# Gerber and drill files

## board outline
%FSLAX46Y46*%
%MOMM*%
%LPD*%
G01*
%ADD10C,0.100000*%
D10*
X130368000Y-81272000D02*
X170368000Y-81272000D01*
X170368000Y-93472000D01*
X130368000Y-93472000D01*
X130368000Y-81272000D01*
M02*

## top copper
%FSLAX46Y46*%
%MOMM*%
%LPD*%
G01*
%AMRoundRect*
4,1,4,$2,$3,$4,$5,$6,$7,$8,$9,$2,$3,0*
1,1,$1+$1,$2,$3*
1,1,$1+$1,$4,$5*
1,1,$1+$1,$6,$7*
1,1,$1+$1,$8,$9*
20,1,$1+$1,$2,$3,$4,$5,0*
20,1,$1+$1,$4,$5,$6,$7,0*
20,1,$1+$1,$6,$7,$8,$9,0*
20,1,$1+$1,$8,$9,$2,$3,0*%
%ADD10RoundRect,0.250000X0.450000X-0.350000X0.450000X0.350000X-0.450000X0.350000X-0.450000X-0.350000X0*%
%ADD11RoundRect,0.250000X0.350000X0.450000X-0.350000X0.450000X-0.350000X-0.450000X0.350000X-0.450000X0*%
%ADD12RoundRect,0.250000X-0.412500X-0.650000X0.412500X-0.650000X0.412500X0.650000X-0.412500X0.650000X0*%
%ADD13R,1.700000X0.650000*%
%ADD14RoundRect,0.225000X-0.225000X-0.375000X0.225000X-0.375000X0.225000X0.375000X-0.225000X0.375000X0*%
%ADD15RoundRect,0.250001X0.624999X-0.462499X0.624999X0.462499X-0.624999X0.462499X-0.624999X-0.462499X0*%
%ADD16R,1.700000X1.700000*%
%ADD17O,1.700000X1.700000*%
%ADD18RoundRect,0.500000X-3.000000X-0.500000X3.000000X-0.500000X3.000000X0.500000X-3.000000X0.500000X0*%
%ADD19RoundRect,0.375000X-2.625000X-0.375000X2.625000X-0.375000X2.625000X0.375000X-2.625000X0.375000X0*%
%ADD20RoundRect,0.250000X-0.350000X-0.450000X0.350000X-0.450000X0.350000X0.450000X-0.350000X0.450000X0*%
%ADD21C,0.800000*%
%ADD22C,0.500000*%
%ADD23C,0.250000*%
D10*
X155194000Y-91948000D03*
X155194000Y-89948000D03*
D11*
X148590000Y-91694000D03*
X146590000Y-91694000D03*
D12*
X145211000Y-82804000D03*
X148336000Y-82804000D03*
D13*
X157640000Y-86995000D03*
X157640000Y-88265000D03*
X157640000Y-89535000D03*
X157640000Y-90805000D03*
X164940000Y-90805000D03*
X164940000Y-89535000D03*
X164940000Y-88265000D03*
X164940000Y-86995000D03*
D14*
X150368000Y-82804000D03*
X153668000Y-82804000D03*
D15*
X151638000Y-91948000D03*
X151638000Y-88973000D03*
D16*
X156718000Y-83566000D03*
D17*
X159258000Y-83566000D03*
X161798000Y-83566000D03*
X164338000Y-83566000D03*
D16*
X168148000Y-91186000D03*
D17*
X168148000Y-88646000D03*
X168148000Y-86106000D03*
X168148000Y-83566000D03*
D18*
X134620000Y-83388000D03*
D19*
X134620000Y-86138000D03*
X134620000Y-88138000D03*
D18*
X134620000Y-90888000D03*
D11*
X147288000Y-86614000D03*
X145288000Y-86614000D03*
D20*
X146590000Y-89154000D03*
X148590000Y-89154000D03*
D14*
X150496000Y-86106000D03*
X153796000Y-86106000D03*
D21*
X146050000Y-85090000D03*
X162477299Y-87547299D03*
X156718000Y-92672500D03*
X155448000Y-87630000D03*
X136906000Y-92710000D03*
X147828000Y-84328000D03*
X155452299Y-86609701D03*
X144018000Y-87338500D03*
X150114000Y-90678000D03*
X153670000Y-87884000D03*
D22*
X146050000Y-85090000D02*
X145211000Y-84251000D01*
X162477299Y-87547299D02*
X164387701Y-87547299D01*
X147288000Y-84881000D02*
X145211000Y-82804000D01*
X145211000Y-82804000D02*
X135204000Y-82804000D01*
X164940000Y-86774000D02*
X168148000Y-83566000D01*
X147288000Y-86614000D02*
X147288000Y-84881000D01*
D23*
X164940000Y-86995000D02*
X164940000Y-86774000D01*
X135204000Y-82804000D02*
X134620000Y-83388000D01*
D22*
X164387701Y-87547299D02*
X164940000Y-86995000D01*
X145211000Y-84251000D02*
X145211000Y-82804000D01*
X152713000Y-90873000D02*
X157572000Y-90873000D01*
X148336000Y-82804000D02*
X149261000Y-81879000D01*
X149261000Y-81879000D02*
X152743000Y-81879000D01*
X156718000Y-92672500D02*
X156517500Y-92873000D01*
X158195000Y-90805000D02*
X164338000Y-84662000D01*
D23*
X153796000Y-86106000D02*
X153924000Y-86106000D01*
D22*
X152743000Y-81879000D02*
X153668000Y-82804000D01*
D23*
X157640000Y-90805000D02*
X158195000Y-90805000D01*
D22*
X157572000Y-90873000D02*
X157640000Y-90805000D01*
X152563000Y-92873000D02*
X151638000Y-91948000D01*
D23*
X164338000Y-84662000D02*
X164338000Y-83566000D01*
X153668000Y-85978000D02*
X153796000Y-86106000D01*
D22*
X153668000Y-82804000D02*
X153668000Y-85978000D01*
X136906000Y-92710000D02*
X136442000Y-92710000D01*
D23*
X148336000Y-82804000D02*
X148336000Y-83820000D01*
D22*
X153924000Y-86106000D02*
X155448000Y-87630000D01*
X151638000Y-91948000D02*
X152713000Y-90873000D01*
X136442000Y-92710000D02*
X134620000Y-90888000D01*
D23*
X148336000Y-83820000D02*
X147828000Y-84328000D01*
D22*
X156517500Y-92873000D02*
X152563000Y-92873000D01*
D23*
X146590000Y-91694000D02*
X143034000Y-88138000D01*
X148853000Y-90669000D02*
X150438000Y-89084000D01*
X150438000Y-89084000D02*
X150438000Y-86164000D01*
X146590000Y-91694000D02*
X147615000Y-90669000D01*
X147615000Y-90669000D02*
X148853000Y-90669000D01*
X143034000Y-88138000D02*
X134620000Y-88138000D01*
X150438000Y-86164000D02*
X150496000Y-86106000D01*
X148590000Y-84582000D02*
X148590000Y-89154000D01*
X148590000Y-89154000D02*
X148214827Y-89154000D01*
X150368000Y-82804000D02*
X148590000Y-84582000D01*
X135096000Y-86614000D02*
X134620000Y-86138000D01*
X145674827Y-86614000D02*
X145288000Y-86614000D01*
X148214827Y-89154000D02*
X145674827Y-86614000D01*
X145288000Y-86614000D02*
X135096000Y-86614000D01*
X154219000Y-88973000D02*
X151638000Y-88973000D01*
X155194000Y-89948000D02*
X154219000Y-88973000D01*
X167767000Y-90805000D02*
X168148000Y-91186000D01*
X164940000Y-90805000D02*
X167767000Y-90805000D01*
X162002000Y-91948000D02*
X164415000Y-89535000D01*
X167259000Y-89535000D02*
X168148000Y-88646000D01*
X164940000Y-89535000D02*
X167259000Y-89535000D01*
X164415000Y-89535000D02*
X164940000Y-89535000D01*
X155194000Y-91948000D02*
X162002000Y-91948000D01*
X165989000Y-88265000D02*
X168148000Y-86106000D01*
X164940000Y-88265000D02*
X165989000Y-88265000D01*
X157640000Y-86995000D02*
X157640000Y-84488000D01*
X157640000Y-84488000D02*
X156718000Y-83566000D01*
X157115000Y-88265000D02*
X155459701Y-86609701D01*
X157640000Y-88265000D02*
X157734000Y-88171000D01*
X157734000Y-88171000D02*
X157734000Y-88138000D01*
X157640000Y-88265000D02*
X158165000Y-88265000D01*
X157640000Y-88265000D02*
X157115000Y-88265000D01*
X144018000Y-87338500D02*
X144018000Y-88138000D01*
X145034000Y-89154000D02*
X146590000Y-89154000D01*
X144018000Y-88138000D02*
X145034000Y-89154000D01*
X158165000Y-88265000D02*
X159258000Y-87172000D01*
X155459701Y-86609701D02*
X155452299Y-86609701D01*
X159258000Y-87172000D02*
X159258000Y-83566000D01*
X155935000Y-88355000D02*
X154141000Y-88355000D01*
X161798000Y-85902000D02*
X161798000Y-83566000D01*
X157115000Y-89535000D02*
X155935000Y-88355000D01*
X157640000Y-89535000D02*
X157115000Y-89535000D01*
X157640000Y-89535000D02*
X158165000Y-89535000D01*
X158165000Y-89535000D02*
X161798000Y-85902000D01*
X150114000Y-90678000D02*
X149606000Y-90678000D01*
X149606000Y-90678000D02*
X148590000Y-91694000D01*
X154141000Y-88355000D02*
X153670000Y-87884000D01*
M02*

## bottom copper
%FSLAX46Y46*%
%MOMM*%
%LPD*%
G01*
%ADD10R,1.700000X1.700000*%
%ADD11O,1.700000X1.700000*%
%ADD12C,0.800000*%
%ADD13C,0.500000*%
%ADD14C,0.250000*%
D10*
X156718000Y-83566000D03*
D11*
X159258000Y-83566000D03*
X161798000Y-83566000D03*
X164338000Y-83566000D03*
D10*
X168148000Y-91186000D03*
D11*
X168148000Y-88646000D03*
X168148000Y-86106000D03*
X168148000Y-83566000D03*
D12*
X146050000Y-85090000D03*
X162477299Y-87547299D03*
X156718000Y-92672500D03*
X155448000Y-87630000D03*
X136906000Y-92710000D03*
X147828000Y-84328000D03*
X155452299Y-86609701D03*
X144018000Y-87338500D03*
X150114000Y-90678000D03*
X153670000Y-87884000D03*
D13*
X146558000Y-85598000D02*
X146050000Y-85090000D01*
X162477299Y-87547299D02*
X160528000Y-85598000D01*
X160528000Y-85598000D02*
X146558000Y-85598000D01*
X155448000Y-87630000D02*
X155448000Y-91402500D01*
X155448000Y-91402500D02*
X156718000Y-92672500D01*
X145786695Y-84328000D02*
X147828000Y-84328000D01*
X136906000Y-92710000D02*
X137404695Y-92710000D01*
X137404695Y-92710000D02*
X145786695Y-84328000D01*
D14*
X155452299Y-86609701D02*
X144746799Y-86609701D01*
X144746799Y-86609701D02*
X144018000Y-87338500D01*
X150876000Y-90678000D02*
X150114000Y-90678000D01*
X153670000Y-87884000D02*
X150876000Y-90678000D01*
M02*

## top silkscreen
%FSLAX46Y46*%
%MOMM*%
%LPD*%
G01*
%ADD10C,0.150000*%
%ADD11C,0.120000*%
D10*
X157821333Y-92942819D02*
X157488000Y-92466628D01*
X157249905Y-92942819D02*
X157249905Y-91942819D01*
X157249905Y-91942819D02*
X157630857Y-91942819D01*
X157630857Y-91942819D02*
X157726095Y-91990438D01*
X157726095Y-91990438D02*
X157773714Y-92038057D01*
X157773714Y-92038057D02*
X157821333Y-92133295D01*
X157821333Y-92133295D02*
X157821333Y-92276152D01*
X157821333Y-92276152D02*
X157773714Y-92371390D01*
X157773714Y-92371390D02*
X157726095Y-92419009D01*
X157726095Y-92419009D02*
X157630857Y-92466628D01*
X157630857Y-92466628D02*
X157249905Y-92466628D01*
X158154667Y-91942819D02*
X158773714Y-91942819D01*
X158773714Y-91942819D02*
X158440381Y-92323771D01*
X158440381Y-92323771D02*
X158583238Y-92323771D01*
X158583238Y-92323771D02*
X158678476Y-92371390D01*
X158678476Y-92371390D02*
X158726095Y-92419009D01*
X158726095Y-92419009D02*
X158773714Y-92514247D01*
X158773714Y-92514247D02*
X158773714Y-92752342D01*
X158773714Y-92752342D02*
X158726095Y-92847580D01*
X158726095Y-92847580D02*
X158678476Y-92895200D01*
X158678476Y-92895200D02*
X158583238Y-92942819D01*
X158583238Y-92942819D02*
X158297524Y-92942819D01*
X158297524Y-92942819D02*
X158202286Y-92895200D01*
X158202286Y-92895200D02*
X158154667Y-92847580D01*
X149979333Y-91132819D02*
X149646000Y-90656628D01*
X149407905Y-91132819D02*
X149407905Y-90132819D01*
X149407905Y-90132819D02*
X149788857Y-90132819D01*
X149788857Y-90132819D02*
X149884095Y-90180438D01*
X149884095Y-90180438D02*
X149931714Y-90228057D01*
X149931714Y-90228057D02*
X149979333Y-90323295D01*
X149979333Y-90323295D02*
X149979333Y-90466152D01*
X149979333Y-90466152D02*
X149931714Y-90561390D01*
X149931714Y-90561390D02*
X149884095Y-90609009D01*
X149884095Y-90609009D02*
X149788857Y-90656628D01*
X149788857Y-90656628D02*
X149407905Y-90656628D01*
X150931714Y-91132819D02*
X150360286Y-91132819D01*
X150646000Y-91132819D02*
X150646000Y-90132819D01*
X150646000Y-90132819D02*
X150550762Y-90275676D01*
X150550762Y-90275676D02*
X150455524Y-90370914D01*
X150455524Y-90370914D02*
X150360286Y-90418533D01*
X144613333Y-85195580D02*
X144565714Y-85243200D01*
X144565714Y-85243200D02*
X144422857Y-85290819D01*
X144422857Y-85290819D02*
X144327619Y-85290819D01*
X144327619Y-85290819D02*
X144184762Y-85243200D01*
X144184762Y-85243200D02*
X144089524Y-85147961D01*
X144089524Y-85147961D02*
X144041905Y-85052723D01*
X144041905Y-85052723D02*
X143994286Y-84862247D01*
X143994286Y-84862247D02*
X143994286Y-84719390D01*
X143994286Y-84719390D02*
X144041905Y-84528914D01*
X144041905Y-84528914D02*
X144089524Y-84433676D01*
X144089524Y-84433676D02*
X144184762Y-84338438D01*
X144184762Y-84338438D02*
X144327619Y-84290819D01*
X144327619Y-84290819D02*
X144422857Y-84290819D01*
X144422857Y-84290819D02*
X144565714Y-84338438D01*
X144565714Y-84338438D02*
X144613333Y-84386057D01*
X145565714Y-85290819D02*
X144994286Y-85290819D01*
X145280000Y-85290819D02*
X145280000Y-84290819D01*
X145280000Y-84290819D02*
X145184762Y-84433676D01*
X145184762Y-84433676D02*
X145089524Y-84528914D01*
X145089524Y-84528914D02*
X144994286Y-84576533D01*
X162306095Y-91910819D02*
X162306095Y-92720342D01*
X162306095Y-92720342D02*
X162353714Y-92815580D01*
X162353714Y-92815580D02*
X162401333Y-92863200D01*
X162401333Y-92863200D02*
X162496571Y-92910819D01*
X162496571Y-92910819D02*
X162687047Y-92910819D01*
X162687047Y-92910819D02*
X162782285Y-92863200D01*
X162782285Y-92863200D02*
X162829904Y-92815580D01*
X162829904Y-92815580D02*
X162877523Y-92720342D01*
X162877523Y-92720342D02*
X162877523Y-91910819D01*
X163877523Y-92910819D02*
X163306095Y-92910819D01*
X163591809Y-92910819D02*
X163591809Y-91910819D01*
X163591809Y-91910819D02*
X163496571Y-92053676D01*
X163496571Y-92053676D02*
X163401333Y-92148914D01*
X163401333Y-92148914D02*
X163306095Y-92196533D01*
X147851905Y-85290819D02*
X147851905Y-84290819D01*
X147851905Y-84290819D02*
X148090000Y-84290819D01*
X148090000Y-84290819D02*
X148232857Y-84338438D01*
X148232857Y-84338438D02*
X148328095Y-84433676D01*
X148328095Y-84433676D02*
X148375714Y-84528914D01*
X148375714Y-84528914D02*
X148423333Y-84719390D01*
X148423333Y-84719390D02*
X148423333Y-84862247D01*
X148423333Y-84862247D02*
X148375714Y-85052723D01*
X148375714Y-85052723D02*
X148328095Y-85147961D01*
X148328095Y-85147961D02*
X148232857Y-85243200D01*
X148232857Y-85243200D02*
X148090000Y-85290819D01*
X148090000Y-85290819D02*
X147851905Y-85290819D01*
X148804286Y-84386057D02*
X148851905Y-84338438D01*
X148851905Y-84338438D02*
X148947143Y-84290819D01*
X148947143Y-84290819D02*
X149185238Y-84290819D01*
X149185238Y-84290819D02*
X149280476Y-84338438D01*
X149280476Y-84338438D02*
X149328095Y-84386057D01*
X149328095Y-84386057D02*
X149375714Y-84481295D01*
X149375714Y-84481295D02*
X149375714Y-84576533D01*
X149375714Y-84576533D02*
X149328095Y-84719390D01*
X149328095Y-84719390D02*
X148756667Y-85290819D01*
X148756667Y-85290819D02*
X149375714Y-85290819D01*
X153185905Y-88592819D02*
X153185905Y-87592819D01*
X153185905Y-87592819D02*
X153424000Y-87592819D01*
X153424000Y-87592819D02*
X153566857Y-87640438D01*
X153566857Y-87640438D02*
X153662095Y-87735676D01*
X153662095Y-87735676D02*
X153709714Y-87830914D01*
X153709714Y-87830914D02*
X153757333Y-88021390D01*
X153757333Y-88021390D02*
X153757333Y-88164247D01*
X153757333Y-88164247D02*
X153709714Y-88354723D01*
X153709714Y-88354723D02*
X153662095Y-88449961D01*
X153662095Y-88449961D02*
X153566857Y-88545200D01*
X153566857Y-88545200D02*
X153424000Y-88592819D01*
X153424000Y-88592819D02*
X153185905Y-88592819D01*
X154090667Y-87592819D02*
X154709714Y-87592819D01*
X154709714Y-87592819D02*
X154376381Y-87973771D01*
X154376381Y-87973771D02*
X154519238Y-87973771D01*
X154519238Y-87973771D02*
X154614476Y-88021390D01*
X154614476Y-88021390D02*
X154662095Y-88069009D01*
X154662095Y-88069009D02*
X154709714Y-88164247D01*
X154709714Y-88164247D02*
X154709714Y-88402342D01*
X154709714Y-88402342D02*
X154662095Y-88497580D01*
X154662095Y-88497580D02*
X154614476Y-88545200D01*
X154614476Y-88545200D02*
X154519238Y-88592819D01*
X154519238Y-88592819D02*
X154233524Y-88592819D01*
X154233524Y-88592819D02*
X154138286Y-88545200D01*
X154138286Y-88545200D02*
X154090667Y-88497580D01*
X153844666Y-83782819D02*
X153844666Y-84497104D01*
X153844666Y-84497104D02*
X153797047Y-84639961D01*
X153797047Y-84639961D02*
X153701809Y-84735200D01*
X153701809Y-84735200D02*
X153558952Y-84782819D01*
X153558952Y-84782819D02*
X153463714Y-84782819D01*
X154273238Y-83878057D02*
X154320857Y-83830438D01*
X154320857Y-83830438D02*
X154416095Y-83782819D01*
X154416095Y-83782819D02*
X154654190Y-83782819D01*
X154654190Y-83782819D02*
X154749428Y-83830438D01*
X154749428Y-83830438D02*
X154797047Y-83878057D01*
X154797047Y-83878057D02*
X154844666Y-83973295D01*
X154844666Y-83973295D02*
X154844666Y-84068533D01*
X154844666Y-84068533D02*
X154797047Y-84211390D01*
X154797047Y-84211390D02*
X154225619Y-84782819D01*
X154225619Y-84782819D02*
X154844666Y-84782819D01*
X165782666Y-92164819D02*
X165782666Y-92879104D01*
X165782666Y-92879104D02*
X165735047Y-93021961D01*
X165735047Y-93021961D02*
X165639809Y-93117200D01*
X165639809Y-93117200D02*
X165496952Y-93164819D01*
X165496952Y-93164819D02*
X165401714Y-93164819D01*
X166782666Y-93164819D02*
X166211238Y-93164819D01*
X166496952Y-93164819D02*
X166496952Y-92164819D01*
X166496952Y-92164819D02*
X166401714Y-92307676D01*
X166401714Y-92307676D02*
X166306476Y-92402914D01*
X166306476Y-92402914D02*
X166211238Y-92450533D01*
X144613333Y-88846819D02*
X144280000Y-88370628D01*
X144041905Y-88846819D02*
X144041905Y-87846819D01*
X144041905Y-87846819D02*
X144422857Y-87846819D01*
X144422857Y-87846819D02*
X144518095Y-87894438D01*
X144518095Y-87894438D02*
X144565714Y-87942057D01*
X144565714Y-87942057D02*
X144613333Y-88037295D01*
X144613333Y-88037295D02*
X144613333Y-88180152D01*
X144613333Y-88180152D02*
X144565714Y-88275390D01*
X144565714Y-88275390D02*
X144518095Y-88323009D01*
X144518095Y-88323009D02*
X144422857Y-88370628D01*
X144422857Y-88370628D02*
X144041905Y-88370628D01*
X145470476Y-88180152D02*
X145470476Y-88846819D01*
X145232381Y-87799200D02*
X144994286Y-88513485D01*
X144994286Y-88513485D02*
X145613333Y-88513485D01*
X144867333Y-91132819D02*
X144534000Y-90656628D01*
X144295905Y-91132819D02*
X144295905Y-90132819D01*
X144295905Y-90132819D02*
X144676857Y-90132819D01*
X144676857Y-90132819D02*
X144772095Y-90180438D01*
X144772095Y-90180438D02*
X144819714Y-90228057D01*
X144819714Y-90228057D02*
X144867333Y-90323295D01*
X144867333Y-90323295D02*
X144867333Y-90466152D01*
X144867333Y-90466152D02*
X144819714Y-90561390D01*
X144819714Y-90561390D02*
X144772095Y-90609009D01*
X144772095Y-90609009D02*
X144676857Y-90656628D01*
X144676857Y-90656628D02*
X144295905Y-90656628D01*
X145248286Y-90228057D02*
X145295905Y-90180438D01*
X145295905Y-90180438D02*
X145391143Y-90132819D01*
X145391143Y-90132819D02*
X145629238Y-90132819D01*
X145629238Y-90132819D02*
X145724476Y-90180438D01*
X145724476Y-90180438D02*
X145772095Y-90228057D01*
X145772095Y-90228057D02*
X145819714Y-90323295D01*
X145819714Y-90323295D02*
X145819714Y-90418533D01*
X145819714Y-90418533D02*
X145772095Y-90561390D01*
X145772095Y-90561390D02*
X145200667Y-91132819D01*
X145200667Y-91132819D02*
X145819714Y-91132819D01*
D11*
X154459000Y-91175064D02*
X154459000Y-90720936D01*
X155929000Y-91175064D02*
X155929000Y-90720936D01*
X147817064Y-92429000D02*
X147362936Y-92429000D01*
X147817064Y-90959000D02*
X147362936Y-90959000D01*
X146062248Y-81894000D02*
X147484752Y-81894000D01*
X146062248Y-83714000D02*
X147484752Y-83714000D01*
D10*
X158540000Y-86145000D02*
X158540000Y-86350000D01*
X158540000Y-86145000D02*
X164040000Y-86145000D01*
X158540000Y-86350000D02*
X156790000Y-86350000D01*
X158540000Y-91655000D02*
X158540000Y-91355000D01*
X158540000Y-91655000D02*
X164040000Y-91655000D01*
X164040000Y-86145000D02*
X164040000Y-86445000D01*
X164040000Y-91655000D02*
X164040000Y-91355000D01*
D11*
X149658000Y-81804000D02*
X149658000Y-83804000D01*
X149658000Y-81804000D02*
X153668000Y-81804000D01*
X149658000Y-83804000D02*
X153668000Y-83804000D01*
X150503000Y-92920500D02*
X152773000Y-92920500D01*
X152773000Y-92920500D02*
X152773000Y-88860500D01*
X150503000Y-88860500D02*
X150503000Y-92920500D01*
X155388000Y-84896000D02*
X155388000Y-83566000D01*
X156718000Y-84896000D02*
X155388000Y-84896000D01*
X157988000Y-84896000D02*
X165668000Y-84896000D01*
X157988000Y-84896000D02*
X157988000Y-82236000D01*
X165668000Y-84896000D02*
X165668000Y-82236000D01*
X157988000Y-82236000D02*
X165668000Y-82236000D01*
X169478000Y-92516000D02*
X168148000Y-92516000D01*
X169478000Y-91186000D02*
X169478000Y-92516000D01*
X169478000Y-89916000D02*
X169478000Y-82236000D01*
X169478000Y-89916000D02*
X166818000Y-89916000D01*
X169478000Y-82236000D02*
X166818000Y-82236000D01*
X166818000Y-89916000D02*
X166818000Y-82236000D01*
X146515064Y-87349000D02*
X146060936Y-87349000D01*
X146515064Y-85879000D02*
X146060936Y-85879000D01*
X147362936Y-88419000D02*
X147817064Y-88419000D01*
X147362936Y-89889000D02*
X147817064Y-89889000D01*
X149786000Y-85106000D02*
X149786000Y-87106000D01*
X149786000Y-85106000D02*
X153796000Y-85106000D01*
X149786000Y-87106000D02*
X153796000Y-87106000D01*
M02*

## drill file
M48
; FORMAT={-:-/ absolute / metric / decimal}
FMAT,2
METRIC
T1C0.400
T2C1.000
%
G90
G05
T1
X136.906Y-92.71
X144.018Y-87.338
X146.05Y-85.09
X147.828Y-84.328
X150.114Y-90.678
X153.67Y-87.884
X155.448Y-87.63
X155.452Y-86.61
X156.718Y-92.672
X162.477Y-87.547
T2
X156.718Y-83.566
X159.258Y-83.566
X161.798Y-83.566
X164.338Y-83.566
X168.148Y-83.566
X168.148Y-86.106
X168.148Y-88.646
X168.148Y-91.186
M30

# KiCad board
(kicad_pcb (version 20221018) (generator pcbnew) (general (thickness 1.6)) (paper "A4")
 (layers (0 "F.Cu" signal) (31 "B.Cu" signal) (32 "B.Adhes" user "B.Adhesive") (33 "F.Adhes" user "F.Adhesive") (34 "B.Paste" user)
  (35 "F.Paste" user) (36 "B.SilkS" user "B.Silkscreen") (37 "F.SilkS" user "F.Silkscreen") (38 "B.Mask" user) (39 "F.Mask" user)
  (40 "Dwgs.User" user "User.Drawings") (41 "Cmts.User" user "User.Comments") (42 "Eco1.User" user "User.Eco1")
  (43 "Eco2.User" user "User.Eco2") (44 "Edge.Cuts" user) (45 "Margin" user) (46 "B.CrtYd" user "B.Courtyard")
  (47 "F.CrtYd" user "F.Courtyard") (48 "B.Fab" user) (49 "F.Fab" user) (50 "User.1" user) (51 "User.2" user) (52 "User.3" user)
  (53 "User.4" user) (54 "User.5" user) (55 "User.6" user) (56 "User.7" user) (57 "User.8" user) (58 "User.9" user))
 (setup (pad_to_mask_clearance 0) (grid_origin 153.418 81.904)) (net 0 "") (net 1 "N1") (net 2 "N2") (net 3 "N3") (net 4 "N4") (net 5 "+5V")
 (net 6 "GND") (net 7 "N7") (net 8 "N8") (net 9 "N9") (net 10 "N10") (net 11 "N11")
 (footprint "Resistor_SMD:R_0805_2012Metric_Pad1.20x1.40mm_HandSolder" (layer "F.Cu") (at 155.194 90.948 90)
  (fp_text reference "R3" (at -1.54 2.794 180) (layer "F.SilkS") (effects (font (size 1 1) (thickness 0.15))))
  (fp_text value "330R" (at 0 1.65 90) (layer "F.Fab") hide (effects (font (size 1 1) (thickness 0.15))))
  (fp_line (start -0.227064 -0.735) (end 0.227064 -0.735) (stroke (width 0.12) (type solid)) (layer "F.SilkS"))
  (fp_line (start -0.227064 0.735) (end 0.227064 0.735) (stroke (width 0.12) (type solid)) (layer "F.SilkS"))
  (pad "1" smd roundrect (at -1 0 90) (size 1.2 1.4) (layers "F.Cu" "F.Paste" "F.Mask") (roundrect_rratio 0.208333) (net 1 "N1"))
  (pad "2" smd roundrect (at 1 0 90) (size 1.2 1.4) (layers "F.Cu" "F.Paste" "F.Mask") (roundrect_rratio 0.208333) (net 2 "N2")))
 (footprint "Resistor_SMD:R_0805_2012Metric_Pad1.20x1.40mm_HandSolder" (layer "F.Cu") (at 147.59 91.694 180)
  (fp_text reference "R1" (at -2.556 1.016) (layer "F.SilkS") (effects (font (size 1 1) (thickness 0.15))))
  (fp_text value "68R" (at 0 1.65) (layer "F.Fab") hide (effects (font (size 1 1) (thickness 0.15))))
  (fp_line (start -0.227064 -0.735) (end 0.227064 -0.735) (stroke (width 0.12) (type solid)) (layer "F.SilkS"))
  (fp_line (start -0.227064 0.735) (end 0.227064 0.735) (stroke (width 0.12) (type solid)) (layer "F.SilkS"))
  (pad "1" smd roundrect (at -1 0 180) (size 1.2 1.4) (layers "F.Cu" "F.Paste" "F.Mask") (roundrect_rratio 0.208333) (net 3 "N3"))
  (pad "2" smd roundrect (at 1 0 180) (size 1.2 1.4) (layers "F.Cu" "F.Paste" "F.Mask") (roundrect_rratio 0.208333) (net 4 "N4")))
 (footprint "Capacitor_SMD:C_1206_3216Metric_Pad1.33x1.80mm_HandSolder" (layer "F.Cu") (at 146.7735 82.804)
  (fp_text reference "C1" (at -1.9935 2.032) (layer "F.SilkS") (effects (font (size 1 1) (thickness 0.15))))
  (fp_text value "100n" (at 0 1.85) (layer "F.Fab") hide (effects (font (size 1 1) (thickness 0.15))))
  (fp_line (start -0.711252 -0.91) (end 0.711252 -0.91) (stroke (width 0.12) (type solid)) (layer "F.SilkS"))
  (fp_line (start -0.711252 0.91) (end 0.711252 0.91) (stroke (width 0.12) (type solid)) (layer "F.SilkS"))
  (pad "1" smd roundrect (at -1.5625 0) (size 1.325 1.8) (layers "F.Cu" "F.Paste" "F.Mask") (roundrect_rratio 0.188679) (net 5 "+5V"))
  (pad "2" smd roundrect (at 1.5625 0) (size 1.325 1.8) (layers "F.Cu" "F.Paste" "F.Mask") (roundrect_rratio 0.188679) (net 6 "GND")))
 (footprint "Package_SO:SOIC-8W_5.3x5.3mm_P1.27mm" (layer "F.Cu") (at 161.29 88.9)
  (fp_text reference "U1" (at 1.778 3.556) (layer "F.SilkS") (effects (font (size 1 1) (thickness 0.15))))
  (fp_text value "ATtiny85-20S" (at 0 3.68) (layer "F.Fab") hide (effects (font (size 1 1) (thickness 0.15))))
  (fp_line (start -2.75 -2.755) (end -2.75 -2.55) (stroke (width 0.15) (type solid)) (layer "F.SilkS"))
  (fp_line (start -2.75 -2.755) (end 2.75 -2.755) (stroke (width 0.15) (type solid)) (layer "F.SilkS"))
  (fp_line (start -2.75 -2.55) (end -4.5 -2.55) (stroke (width 0.15) (type solid)) (layer "F.SilkS"))
  (fp_line (start -2.75 2.755) (end -2.75 2.455) (stroke (width 0.15) (type solid)) (layer "F.SilkS"))
  (fp_line (start -2.75 2.755) (end 2.75 2.755) (stroke (width 0.15) (type solid)) (layer "F.SilkS"))
  (fp_line (start 2.75 -2.755) (end 2.75 -2.455) (stroke (width 0.15) (type solid)) (layer "F.SilkS"))
  (fp_line (start 2.75 2.755) (end 2.75 2.455) (stroke (width 0.15) (type solid)) (layer "F.SilkS"))
  (pad "1" smd rect (at -3.65 -1.905) (size 1.7 0.65) (layers "F.Cu" "F.Paste" "F.Mask") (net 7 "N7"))
  (pad "2" smd rect (at -3.65 -0.635) (size 1.7 0.65) (layers "F.Cu" "F.Paste" "F.Mask") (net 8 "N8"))
  (pad "3" smd rect (at -3.65 0.635) (size 1.7 0.65) (layers "F.Cu" "F.Paste" "F.Mask") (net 3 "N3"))
  (pad "4" smd rect (at -3.65 1.905) (size 1.7 0.65) (layers "F.Cu" "F.Paste" "F.Mask") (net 6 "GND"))
  (pad "5" smd rect (at 3.65 1.905) (size 1.7 0.65) (layers "F.Cu" "F.Paste" "F.Mask") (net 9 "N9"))
  (pad "6" smd rect (at 3.65 0.635) (size 1.7 0.65) (layers "F.Cu" "F.Paste" "F.Mask") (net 1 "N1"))
  (pad "7" smd rect (at 3.65 -0.635) (size 1.7 0.65) (layers "F.Cu" "F.Paste" "F.Mask") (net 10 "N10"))
  (pad "8" smd rect (at 3.65 -1.905) (size 1.7 0.65) (layers "F.Cu" "F.Paste" "F.Mask") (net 5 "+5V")))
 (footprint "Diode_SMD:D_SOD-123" (layer "F.Cu") (at 152.018 82.804)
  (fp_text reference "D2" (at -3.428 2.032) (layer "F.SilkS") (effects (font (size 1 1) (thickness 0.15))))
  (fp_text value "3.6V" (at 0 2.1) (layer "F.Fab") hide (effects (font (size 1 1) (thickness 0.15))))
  (fp_line (start -2.36 -1) (end -2.36 1) (stroke (width 0.12) (type solid)) (layer "F.SilkS"))
  (fp_line (start -2.36 -1) (end 1.65 -1) (stroke (width 0.12) (type solid)) (layer "F.SilkS"))
  (fp_line (start -2.36 1) (end 1.65 1) (stroke (width 0.12) (type solid)) (layer "F.SilkS"))
  (pad "1" smd roundrect (at -1.65 0) (size 0.9 1.2) (layers "F.Cu" "F.Paste" "F.Mask") (roundrect_rratio 0.25) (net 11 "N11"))
  (pad "2" smd roundrect (at 1.65 0) (size 0.9 1.2) (layers "F.Cu" "F.Paste" "F.Mask") (roundrect_rratio 0.25) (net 6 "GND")))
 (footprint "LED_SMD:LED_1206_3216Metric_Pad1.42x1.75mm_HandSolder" (layer "F.Cu") (at 151.638 90.4605 90)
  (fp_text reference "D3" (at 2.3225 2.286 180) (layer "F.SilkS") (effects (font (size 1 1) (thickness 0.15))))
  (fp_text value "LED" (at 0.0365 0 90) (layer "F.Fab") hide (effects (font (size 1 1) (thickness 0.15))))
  (fp_line (start -2.46 -1.135) (end -2.46 1.135) (stroke (width 0.12) (type solid)) (layer "F.SilkS"))
  (fp_line (start -2.46 1.135) (end 1.6 1.135) (stroke (width 0.12) (type solid)) (layer "F.SilkS"))
  (fp_line (start 1.6 -1.135) (end -2.46 -1.135) (stroke (width 0.12) (type solid)) (layer "F.SilkS"))
  (pad "1" smd roundrect (at -1.4875 0 90) (size 1.425 1.75) (layers "F.Cu" "F.Paste" "F.Mask") (roundrect_rratio 0.175439) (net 6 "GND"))
  (pad "2" smd roundrect (at 1.4875 0 90) (size 1.425 1.75) (layers "F.Cu" "F.Paste" "F.Mask") (roundrect_rratio 0.175439) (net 2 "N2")))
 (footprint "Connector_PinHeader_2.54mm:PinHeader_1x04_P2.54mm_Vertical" (layer "F.Cu") (at 156.718 83.566 90)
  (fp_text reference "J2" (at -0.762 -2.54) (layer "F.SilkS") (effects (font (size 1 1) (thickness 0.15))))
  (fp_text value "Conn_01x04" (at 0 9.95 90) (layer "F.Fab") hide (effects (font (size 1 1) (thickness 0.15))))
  (fp_line (start -1.33 -1.33) (end 0 -1.33) (stroke (width 0.12) (type solid)) (layer "F.SilkS"))
  (fp_line (start -1.33 0) (end -1.33 -1.33) (stroke (width 0.12) (type solid)) (layer "F.SilkS"))
  (fp_line (start -1.33 1.27) (end -1.33 8.95) (stroke (width 0.12) (type solid)) (layer "F.SilkS"))
  (fp_line (start -1.33 1.27) (end 1.33 1.27) (stroke (width 0.12) (type solid)) (layer "F.SilkS"))
  (fp_line (start -1.33 8.95) (end 1.33 8.95) (stroke (width 0.12) (type solid)) (layer "F.SilkS"))
  (fp_line (start 1.33 1.27) (end 1.33 8.95) (stroke (width 0.12) (type solid)) (layer "F.SilkS"))
  (pad "1" thru_hole rect (at 0 0 90) (size 1.7 1.7) (drill 1) (layers "*.Cu" "*.Mask") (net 7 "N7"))
  (pad "2" thru_hole oval (at 0 2.54 90) (size 1.7 1.7) (drill 1) (layers "*.Cu" "*.Mask") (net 8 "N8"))
  (pad "3" thru_hole oval (at 0 5.08 90) (size 1.7 1.7) (drill 1) (layers "*.Cu" "*.Mask") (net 3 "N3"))
  (pad "4" thru_hole oval (at 0 7.62 90) (size 1.7 1.7) (drill 1) (layers "*.Cu" "*.Mask") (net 6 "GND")))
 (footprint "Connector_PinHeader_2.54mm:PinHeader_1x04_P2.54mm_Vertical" (layer "F.Cu") (at 168.148 91.186 180)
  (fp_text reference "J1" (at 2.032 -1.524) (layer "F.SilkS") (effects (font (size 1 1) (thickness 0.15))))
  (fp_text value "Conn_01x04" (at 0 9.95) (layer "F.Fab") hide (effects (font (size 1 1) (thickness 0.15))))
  (fp_line (start -1.33 -1.33) (end 0 -1.33) (stroke (width 0.12) (type solid)) (layer "F.SilkS"))
  (fp_line (start -1.33 0) (end -1.33 -1.33) (stroke (width 0.12) (type solid)) (layer "F.SilkS"))
  (fp_line (start -1.33 1.27) (end -1.33 8.95) (stroke (width 0.12) (type solid)) (layer "F.SilkS"))
  (fp_line (start -1.33 1.27) (end 1.33 1.27) (stroke (width 0.12) (type solid)) (layer "F.SilkS"))
  (fp_line (start -1.33 8.95) (end 1.33 8.95) (stroke (width 0.12) (type solid)) (layer "F.SilkS"))
  (fp_line (start 1.33 1.27) (end 1.33 8.95) (stroke (width 0.12) (type solid)) (layer "F.SilkS"))
  (pad "1" thru_hole rect (at 0 0 180) (size 1.7 1.7) (drill 1) (layers "*.Cu" "*.Mask") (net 9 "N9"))
  (pad "2" thru_hole oval (at 0 2.54 180) (size 1.7 1.7) (drill 1) (layers "*.Cu" "*.Mask") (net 1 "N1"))
  (pad "3" thru_hole oval (at 0 5.08 180) (size 1.7 1.7) (drill 1) (layers "*.Cu" "*.Mask") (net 10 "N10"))
  (pad "4" thru_hole oval (at 0 7.62 180) (size 1.7 1.7) (drill 1) (layers "*.Cu" "*.Mask") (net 5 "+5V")))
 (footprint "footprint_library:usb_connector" (layer "F.Cu") (at 134.62 87.138)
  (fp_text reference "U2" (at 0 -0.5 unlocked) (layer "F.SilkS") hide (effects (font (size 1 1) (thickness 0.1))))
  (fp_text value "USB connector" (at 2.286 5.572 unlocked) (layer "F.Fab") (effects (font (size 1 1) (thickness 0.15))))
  (pad "1" smd roundrect (at 0 -3.75) (size 7 2) (layers "F.Cu" "F.Paste" "F.Mask") (roundrect_rratio 0.25) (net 5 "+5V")
   (thermal_bridge_angle 45))
  (pad "2" smd roundrect (at 0 -1) (size 6 1.5) (layers "F.Cu" "F.Paste" "F.Mask") (roundrect_rratio 0.25) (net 11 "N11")
   (thermal_bridge_angle 45))
  (pad "3" smd roundrect (at 0 1) (size 6 1.5) (layers "F.Cu" "F.Paste" "F.Mask") (roundrect_rratio 0.25) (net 4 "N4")
   (thermal_bridge_angle 45))
  (pad "4" smd roundrect (at 0 3.75) (size 7 2) (layers "F.Cu" "F.Paste" "F.Mask") (roundrect_rratio 0.25) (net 6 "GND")
   (thermal_bridge_angle 45)))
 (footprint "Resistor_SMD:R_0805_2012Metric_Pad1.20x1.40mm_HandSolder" (layer "F.Cu") (at 146.288 86.614 180)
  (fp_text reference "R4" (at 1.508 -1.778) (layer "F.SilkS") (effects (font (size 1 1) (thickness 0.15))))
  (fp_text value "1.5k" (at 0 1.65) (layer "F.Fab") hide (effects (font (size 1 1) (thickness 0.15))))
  (fp_line (start -0.227064 -0.735) (end 0.227064 -0.735) (stroke (width 0.12) (type solid)) (layer "F.SilkS"))
  (fp_line (start -0.227064 0.735) (end 0.227064 0.735) (stroke (width 0.12) (type solid)) (layer "F.SilkS"))
  (pad "1" smd roundrect (at -1 0 180) (size 1.2 1.4) (layers "F.Cu" "F.Paste" "F.Mask") (roundrect_rratio 0.208333) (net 5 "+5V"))
  (pad "2" smd roundrect (at 1 0 180) (size 1.2 1.4) (layers "F.Cu" "F.Paste" "F.Mask") (roundrect_rratio 0.208333) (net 11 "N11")))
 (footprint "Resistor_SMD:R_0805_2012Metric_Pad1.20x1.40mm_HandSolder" (layer "F.Cu") (at 147.59 89.154)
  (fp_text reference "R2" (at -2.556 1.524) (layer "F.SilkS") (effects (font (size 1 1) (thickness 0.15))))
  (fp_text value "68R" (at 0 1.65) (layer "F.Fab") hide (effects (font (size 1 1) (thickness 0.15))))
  (fp_line (start -0.227064 -0.735) (end 0.227064 -0.735) (stroke (width 0.12) (type solid)) (layer "F.SilkS"))
  (fp_line (start -0.227064 0.735) (end 0.227064 0.735) (stroke (width 0.12) (type solid)) (layer "F.SilkS"))
  (pad "1" smd roundrect (at -1 0) (size 1.2 1.4) (layers "F.Cu" "F.Paste" "F.Mask") (roundrect_rratio 0.208333) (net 8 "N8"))
  (pad "2" smd roundrect (at 1 0) (size 1.2 1.4) (layers "F.Cu" "F.Paste" "F.Mask") (roundrect_rratio 0.208333) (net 11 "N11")))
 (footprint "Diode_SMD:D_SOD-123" (layer "F.Cu") (at 152.146 86.106)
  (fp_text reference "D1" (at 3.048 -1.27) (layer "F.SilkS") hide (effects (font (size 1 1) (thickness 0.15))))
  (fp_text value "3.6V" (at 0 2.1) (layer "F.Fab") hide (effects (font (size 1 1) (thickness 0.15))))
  (fp_line (start -2.36 -1) (end -2.36 1) (stroke (width 0.12) (type solid)) (layer "F.SilkS"))
  (fp_line (start -2.36 -1) (end 1.65 -1) (stroke (width 0.12) (type solid)) (layer "F.SilkS"))
  (fp_line (start -2.36 1) (end 1.65 1) (stroke (width 0.12) (type solid)) (layer "F.SilkS"))
  (pad "1" smd roundrect (at -1.65 0) (size 0.9 1.2) (layers "F.Cu" "F.Paste" "F.Mask") (roundrect_rratio 0.25) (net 4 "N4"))
  (pad "2" smd roundrect (at 1.65 0) (size 0.9 1.2) (layers "F.Cu" "F.Paste" "F.Mask") (roundrect_rratio 0.25) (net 6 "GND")))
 (gr_rect (start 130.368 81.272) (end 170.368 93.472) (stroke (width 0.1) (type default)) (fill none) (layer "Edge.Cuts"))
 (segment (start 146.05 85.09) (end 145.211 84.251) (width 0.5) (layer "F.Cu") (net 5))
 (segment (start 162.477299 87.547299) (end 164.387701 87.547299) (width 0.5) (layer "F.Cu") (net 5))
 (segment (start 147.288 84.881) (end 145.211 82.804) (width 0.5) (layer "F.Cu") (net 5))
 (segment (start 145.211 82.804) (end 135.204 82.804) (width 0.5) (layer "F.Cu") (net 5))
 (segment (start 164.94 86.774) (end 168.148 83.566) (width 0.5) (layer "F.Cu") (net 5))
 (segment (start 147.288 86.614) (end 147.288 84.881) (width 0.5) (layer "F.Cu") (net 5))
 (segment (start 164.94 86.995) (end 164.94 86.774) (width 0.25) (layer "F.Cu") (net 5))
 (segment (start 135.204 82.804) (end 134.62 83.388) (width 0.25) (layer "F.Cu") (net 5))
 (segment (start 164.387701 87.547299) (end 164.94 86.995) (width 0.5) (layer "F.Cu") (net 5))
 (segment (start 145.211 84.251) (end 145.211 82.804) (width 0.5) (layer "F.Cu") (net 5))
 (via (at 146.05 85.09) (size 0.8) (drill 0.4) (layers "F.Cu" "B.Cu") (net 5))
 (via (at 162.477299 87.547299) (size 0.8) (drill 0.4) (layers "F.Cu" "B.Cu") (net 5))
 (segment (start 146.558 85.598) (end 146.05 85.09) (width 0.5) (layer "B.Cu") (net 5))
 (segment (start 162.477299 87.547299) (end 160.528 85.598) (width 0.5) (layer "B.Cu") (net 5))
 (segment (start 160.528 85.598) (end 146.558 85.598) (width 0.5) (layer "B.Cu") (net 5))
 (segment (start 152.713 90.873) (end 157.572 90.873) (width 0.5) (layer "F.Cu") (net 6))
 (segment (start 148.336 82.804) (end 149.261 81.879) (width 0.5) (layer "F.Cu") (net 6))
 (segment (start 149.261 81.879) (end 152.743 81.879) (width 0.5) (layer "F.Cu") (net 6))
 (segment (start 156.718 92.6725) (end 156.5175 92.873) (width 0.5) (layer "F.Cu") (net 6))
 (segment (start 158.195 90.805) (end 164.338 84.662) (width 0.5) (layer "F.Cu") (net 6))
 (segment (start 153.796 86.106) (end 153.924 86.106) (width 0.25) (layer "F.Cu") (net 6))
 (segment (start 152.743 81.879) (end 153.668 82.804) (width 0.5) (layer "F.Cu") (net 6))
 (segment (start 157.64 90.805) (end 158.195 90.805) (width 0.25) (layer "F.Cu") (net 6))
 (segment (start 157.572 90.873) (end 157.64 90.805) (width 0.5) (layer "F.Cu") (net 6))
 (segment (start 152.563 92.873) (end 151.638 91.948) (width 0.5) (layer "F.Cu") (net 6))
 (segment (start 164.338 84.662) (end 164.338 83.566) (width 0.25) (layer "F.Cu") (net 6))
 (segment (start 153.668 85.978) (end 153.796 86.106) (width 0.25) (layer "F.Cu") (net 6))
 (segment (start 153.668 82.804) (end 153.668 85.978) (width 0.5) (layer "F.Cu") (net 6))
 (segment (start 136.906 92.71) (end 136.442 92.71) (width 0.5) (layer "F.Cu") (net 6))
 (segment (start 148.336 82.804) (end 148.336 83.82) (width 0.25) (layer "F.Cu") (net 6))
 (segment (start 153.924 86.106) (end 155.448 87.63) (width 0.5) (layer "F.Cu") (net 6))
 (segment (start 151.638 91.948) (end 152.713 90.873) (width 0.5) (layer "F.Cu") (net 6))
 (segment (start 136.442 92.71) (end 134.62 90.888) (width 0.5) (layer "F.Cu") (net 6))
 (segment (start 148.336 83.82) (end 147.828 84.328) (width 0.25) (layer "F.Cu") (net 6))
 (segment (start 156.5175 92.873) (end 152.563 92.873) (width 0.5) (layer "F.Cu") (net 6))
 (via (at 156.718 92.6725) (size 0.8) (drill 0.4) (layers "F.Cu" "B.Cu") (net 6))
 (via (at 155.448 87.63) (size 0.8) (drill 0.4) (layers "F.Cu" "B.Cu") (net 6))
 (via (at 136.906 92.71) (size 0.8) (drill 0.4) (layers "F.Cu" "B.Cu") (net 6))
 (via (at 147.828 84.328) (size 0.8) (drill 0.4) (layers "F.Cu" "B.Cu") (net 6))
 (segment (start 155.448 87.63) (end 155.448 91.4025) (width 0.5) (layer "B.Cu") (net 6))
 (segment (start 155.448 91.4025) (end 156.718 92.6725) (width 0.5) (layer "B.Cu") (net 6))
 (segment (start 145.786695 84.328) (end 147.828 84.328) (width 0.5) (layer "B.Cu") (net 6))
 (segment (start 136.906 92.71) (end 137.404695 92.71) (width 0.5) (layer "B.Cu") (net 6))
 (segment (start 137.404695 92.71) (end 145.786695 84.328) (width 0.5) (layer "B.Cu") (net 6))
 (segment (start 146.59 91.694) (end 143.034 88.138) (width 0.25) (layer "F.Cu") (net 4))
 (segment (start 148.853 90.669) (end 150.438 89.084) (width 0.25) (layer "F.Cu") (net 4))
 (segment (start 150.438 89.084) (end 150.438 86.164) (width 0.25) (layer "F.Cu") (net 4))
 (segment (start 146.59 91.694) (end 147.615 90.669) (width 0.25) (layer "F.Cu") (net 4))
 (segment (start 147.615 90.669) (end 148.853 90.669) (width 0.25) (layer "F.Cu") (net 4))
 (segment (start 143.034 88.138) (end 134.62 88.138) (width 0.25) (layer "F.Cu") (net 4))
 (segment (start 150.438 86.164) (end 150.496 86.106) (width 0.25) (layer "F.Cu") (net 4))
 (segment (start 148.59 84.582) (end 148.59 89.154) (width 0.25) (layer "F.Cu") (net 11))
 (segment (start 148.59 89.154) (end 148.214827 89.154) (width 0.25) (layer "F.Cu") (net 11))
 (segment (start 150.368 82.804) (end 148.59 84.582) (width 0.25) (layer "F.Cu") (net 11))
 (segment (start 135.096 86.614) (end 134.62 86.138) (width 0.25) (layer "F.Cu") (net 11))
 (segment (start 145.674827 86.614) (end 145.288 86.614) (width 0.25) (layer "F.Cu") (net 11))
 (segment (start 148.214827 89.154) (end 145.674827 86.614) (width 0.25) (layer "F.Cu") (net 11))
 (segment (start 145.288 86.614) (end 135.096 86.614) (width 0.25) (layer "F.Cu") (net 11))
 (segment (start 154.219 88.973) (end 151.638 88.973) (width 0.25) (layer "F.Cu") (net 2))
 (segment (start 155.194 89.948) (end 154.219 88.973) (width 0.25) (layer "F.Cu") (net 2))
 (segment (start 167.767 90.805) (end 168.148 91.186) (width 0.25) (layer "F.Cu") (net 9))
 (segment (start 164.94 90.805) (end 167.767 90.805) (width 0.25) (layer "F.Cu") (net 9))
 (segment (start 162.002 91.948) (end 164.415 89.535) (width 0.25) (layer "F.Cu") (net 1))
 (segment (start 167.259 89.535) (end 168.148 88.646) (width 0.25) (layer "F.Cu") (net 1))
 (segment (start 164.94 89.535) (end 167.259 89.535) (width 0.25) (layer "F.Cu") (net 1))
 (segment (start 164.415 89.535) (end 164.94 89.535) (width 0.25) (layer "F.Cu") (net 1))
 (segment (start 155.194 91.948) (end 162.002 91.948) (width 0.25) (layer "F.Cu") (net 1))
 (segment (start 165.989 88.265) (end 168.148 86.106) (width 0.25) (layer "F.Cu") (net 10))
 (segment (start 164.94 88.265) (end 165.989 88.265) (width 0.25) (layer "F.Cu") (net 10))
 (segment (start 157.64 86.995) (end 157.64 84.488) (width 0.25) (layer "F.Cu") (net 7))
 (segment (start 157.64 84.488) (end 156.718 83.566) (width 0.25) (layer "F.Cu") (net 7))
 (segment (start 157.115 88.265) (end 155.459701 86.609701) (width 0.25) (layer "F.Cu") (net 8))
 (segment (start 157.64 88.265) (end 157.734 88.171) (width 0.25) (layer "F.Cu") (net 8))
 (segment (start 157.734 88.171) (end 157.734 88.138) (width 0.25) (layer "F.Cu") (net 8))
 (segment (start 157.64 88.265) (end 158.165 88.265) (width 0.25) (layer "F.Cu") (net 8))
 (segment (start 157.64 88.265) (end 157.115 88.265) (width 0.25) (layer "F.Cu") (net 8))
 (segment (start 144.018 87.3385) (end 144.018 88.138) (width 0.25) (layer "F.Cu") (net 8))
 (segment (start 145.034 89.154) (end 146.59 89.154) (width 0.25) (layer "F.Cu") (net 8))
 (segment (start 144.018 88.138) (end 145.034 89.154) (width 0.25) (layer "F.Cu") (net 8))
 (segment (start 158.165 88.265) (end 159.258 87.172) (width 0.25) (layer "F.Cu") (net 8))
 (segment (start 155.459701 86.609701) (end 155.452299 86.609701) (width 0.25) (layer "F.Cu") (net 8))
 (segment (start 159.258 87.172) (end 159.258 83.566) (width 0.25) (layer "F.Cu") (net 8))
 (via (at 155.452299 86.609701) (size 0.8) (drill 0.4) (layers "F.Cu" "B.Cu") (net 8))
 (via (at 144.018 87.3385) (size 0.8) (drill 0.4) (layers "F.Cu" "B.Cu") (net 8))
 (segment (start 155.452299 86.609701) (end 144.746799 86.609701) (width 0.25) (layer "B.Cu") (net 8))
 (segment (start 144.746799 86.609701) (end 144.018 87.3385) (width 0.25) (layer "B.Cu") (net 8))
 (segment (start 155.935 88.355) (end 154.141 88.355) (width 0.25) (layer "F.Cu") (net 3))
 (segment (start 161.798 85.902) (end 161.798 83.566) (width 0.25) (layer "F.Cu") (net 3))
 (segment (start 157.115 89.535) (end 155.935 88.355) (width 0.25) (layer "F.Cu") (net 3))
 (segment (start 157.64 89.535) (end 157.115 89.535) (width 0.25) (layer "F.Cu") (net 3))
 (segment (start 157.64 89.535) (end 158.165 89.535) (width 0.25) (layer "F.Cu") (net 3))
 (segment (start 158.165 89.535) (end 161.798 85.902) (width 0.25) (layer "F.Cu") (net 3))
 (segment (start 150.114 90.678) (end 149.606 90.678) (width 0.25) (layer "F.Cu") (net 3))
 (segment (start 149.606 90.678) (end 148.59 91.694) (width 0.25) (layer "F.Cu") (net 3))
 (segment (start 154.141 88.355) (end 153.67 87.884) (width 0.25) (layer "F.Cu") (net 3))
 (via (at 150.114 90.678) (size 0.8) (drill 0.4) (layers "F.Cu" "B.Cu") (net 3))
 (via (at 153.67 87.884) (size 0.8) (drill 0.4) (layers "F.Cu" "B.Cu") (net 3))
 (segment (start 150.876 90.678) (end 150.114 90.678) (width 0.25) (layer "B.Cu") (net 3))
 (segment (start 153.67 87.884) (end 150.876 90.678) (width 0.25) (layer "B.Cu") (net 3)))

